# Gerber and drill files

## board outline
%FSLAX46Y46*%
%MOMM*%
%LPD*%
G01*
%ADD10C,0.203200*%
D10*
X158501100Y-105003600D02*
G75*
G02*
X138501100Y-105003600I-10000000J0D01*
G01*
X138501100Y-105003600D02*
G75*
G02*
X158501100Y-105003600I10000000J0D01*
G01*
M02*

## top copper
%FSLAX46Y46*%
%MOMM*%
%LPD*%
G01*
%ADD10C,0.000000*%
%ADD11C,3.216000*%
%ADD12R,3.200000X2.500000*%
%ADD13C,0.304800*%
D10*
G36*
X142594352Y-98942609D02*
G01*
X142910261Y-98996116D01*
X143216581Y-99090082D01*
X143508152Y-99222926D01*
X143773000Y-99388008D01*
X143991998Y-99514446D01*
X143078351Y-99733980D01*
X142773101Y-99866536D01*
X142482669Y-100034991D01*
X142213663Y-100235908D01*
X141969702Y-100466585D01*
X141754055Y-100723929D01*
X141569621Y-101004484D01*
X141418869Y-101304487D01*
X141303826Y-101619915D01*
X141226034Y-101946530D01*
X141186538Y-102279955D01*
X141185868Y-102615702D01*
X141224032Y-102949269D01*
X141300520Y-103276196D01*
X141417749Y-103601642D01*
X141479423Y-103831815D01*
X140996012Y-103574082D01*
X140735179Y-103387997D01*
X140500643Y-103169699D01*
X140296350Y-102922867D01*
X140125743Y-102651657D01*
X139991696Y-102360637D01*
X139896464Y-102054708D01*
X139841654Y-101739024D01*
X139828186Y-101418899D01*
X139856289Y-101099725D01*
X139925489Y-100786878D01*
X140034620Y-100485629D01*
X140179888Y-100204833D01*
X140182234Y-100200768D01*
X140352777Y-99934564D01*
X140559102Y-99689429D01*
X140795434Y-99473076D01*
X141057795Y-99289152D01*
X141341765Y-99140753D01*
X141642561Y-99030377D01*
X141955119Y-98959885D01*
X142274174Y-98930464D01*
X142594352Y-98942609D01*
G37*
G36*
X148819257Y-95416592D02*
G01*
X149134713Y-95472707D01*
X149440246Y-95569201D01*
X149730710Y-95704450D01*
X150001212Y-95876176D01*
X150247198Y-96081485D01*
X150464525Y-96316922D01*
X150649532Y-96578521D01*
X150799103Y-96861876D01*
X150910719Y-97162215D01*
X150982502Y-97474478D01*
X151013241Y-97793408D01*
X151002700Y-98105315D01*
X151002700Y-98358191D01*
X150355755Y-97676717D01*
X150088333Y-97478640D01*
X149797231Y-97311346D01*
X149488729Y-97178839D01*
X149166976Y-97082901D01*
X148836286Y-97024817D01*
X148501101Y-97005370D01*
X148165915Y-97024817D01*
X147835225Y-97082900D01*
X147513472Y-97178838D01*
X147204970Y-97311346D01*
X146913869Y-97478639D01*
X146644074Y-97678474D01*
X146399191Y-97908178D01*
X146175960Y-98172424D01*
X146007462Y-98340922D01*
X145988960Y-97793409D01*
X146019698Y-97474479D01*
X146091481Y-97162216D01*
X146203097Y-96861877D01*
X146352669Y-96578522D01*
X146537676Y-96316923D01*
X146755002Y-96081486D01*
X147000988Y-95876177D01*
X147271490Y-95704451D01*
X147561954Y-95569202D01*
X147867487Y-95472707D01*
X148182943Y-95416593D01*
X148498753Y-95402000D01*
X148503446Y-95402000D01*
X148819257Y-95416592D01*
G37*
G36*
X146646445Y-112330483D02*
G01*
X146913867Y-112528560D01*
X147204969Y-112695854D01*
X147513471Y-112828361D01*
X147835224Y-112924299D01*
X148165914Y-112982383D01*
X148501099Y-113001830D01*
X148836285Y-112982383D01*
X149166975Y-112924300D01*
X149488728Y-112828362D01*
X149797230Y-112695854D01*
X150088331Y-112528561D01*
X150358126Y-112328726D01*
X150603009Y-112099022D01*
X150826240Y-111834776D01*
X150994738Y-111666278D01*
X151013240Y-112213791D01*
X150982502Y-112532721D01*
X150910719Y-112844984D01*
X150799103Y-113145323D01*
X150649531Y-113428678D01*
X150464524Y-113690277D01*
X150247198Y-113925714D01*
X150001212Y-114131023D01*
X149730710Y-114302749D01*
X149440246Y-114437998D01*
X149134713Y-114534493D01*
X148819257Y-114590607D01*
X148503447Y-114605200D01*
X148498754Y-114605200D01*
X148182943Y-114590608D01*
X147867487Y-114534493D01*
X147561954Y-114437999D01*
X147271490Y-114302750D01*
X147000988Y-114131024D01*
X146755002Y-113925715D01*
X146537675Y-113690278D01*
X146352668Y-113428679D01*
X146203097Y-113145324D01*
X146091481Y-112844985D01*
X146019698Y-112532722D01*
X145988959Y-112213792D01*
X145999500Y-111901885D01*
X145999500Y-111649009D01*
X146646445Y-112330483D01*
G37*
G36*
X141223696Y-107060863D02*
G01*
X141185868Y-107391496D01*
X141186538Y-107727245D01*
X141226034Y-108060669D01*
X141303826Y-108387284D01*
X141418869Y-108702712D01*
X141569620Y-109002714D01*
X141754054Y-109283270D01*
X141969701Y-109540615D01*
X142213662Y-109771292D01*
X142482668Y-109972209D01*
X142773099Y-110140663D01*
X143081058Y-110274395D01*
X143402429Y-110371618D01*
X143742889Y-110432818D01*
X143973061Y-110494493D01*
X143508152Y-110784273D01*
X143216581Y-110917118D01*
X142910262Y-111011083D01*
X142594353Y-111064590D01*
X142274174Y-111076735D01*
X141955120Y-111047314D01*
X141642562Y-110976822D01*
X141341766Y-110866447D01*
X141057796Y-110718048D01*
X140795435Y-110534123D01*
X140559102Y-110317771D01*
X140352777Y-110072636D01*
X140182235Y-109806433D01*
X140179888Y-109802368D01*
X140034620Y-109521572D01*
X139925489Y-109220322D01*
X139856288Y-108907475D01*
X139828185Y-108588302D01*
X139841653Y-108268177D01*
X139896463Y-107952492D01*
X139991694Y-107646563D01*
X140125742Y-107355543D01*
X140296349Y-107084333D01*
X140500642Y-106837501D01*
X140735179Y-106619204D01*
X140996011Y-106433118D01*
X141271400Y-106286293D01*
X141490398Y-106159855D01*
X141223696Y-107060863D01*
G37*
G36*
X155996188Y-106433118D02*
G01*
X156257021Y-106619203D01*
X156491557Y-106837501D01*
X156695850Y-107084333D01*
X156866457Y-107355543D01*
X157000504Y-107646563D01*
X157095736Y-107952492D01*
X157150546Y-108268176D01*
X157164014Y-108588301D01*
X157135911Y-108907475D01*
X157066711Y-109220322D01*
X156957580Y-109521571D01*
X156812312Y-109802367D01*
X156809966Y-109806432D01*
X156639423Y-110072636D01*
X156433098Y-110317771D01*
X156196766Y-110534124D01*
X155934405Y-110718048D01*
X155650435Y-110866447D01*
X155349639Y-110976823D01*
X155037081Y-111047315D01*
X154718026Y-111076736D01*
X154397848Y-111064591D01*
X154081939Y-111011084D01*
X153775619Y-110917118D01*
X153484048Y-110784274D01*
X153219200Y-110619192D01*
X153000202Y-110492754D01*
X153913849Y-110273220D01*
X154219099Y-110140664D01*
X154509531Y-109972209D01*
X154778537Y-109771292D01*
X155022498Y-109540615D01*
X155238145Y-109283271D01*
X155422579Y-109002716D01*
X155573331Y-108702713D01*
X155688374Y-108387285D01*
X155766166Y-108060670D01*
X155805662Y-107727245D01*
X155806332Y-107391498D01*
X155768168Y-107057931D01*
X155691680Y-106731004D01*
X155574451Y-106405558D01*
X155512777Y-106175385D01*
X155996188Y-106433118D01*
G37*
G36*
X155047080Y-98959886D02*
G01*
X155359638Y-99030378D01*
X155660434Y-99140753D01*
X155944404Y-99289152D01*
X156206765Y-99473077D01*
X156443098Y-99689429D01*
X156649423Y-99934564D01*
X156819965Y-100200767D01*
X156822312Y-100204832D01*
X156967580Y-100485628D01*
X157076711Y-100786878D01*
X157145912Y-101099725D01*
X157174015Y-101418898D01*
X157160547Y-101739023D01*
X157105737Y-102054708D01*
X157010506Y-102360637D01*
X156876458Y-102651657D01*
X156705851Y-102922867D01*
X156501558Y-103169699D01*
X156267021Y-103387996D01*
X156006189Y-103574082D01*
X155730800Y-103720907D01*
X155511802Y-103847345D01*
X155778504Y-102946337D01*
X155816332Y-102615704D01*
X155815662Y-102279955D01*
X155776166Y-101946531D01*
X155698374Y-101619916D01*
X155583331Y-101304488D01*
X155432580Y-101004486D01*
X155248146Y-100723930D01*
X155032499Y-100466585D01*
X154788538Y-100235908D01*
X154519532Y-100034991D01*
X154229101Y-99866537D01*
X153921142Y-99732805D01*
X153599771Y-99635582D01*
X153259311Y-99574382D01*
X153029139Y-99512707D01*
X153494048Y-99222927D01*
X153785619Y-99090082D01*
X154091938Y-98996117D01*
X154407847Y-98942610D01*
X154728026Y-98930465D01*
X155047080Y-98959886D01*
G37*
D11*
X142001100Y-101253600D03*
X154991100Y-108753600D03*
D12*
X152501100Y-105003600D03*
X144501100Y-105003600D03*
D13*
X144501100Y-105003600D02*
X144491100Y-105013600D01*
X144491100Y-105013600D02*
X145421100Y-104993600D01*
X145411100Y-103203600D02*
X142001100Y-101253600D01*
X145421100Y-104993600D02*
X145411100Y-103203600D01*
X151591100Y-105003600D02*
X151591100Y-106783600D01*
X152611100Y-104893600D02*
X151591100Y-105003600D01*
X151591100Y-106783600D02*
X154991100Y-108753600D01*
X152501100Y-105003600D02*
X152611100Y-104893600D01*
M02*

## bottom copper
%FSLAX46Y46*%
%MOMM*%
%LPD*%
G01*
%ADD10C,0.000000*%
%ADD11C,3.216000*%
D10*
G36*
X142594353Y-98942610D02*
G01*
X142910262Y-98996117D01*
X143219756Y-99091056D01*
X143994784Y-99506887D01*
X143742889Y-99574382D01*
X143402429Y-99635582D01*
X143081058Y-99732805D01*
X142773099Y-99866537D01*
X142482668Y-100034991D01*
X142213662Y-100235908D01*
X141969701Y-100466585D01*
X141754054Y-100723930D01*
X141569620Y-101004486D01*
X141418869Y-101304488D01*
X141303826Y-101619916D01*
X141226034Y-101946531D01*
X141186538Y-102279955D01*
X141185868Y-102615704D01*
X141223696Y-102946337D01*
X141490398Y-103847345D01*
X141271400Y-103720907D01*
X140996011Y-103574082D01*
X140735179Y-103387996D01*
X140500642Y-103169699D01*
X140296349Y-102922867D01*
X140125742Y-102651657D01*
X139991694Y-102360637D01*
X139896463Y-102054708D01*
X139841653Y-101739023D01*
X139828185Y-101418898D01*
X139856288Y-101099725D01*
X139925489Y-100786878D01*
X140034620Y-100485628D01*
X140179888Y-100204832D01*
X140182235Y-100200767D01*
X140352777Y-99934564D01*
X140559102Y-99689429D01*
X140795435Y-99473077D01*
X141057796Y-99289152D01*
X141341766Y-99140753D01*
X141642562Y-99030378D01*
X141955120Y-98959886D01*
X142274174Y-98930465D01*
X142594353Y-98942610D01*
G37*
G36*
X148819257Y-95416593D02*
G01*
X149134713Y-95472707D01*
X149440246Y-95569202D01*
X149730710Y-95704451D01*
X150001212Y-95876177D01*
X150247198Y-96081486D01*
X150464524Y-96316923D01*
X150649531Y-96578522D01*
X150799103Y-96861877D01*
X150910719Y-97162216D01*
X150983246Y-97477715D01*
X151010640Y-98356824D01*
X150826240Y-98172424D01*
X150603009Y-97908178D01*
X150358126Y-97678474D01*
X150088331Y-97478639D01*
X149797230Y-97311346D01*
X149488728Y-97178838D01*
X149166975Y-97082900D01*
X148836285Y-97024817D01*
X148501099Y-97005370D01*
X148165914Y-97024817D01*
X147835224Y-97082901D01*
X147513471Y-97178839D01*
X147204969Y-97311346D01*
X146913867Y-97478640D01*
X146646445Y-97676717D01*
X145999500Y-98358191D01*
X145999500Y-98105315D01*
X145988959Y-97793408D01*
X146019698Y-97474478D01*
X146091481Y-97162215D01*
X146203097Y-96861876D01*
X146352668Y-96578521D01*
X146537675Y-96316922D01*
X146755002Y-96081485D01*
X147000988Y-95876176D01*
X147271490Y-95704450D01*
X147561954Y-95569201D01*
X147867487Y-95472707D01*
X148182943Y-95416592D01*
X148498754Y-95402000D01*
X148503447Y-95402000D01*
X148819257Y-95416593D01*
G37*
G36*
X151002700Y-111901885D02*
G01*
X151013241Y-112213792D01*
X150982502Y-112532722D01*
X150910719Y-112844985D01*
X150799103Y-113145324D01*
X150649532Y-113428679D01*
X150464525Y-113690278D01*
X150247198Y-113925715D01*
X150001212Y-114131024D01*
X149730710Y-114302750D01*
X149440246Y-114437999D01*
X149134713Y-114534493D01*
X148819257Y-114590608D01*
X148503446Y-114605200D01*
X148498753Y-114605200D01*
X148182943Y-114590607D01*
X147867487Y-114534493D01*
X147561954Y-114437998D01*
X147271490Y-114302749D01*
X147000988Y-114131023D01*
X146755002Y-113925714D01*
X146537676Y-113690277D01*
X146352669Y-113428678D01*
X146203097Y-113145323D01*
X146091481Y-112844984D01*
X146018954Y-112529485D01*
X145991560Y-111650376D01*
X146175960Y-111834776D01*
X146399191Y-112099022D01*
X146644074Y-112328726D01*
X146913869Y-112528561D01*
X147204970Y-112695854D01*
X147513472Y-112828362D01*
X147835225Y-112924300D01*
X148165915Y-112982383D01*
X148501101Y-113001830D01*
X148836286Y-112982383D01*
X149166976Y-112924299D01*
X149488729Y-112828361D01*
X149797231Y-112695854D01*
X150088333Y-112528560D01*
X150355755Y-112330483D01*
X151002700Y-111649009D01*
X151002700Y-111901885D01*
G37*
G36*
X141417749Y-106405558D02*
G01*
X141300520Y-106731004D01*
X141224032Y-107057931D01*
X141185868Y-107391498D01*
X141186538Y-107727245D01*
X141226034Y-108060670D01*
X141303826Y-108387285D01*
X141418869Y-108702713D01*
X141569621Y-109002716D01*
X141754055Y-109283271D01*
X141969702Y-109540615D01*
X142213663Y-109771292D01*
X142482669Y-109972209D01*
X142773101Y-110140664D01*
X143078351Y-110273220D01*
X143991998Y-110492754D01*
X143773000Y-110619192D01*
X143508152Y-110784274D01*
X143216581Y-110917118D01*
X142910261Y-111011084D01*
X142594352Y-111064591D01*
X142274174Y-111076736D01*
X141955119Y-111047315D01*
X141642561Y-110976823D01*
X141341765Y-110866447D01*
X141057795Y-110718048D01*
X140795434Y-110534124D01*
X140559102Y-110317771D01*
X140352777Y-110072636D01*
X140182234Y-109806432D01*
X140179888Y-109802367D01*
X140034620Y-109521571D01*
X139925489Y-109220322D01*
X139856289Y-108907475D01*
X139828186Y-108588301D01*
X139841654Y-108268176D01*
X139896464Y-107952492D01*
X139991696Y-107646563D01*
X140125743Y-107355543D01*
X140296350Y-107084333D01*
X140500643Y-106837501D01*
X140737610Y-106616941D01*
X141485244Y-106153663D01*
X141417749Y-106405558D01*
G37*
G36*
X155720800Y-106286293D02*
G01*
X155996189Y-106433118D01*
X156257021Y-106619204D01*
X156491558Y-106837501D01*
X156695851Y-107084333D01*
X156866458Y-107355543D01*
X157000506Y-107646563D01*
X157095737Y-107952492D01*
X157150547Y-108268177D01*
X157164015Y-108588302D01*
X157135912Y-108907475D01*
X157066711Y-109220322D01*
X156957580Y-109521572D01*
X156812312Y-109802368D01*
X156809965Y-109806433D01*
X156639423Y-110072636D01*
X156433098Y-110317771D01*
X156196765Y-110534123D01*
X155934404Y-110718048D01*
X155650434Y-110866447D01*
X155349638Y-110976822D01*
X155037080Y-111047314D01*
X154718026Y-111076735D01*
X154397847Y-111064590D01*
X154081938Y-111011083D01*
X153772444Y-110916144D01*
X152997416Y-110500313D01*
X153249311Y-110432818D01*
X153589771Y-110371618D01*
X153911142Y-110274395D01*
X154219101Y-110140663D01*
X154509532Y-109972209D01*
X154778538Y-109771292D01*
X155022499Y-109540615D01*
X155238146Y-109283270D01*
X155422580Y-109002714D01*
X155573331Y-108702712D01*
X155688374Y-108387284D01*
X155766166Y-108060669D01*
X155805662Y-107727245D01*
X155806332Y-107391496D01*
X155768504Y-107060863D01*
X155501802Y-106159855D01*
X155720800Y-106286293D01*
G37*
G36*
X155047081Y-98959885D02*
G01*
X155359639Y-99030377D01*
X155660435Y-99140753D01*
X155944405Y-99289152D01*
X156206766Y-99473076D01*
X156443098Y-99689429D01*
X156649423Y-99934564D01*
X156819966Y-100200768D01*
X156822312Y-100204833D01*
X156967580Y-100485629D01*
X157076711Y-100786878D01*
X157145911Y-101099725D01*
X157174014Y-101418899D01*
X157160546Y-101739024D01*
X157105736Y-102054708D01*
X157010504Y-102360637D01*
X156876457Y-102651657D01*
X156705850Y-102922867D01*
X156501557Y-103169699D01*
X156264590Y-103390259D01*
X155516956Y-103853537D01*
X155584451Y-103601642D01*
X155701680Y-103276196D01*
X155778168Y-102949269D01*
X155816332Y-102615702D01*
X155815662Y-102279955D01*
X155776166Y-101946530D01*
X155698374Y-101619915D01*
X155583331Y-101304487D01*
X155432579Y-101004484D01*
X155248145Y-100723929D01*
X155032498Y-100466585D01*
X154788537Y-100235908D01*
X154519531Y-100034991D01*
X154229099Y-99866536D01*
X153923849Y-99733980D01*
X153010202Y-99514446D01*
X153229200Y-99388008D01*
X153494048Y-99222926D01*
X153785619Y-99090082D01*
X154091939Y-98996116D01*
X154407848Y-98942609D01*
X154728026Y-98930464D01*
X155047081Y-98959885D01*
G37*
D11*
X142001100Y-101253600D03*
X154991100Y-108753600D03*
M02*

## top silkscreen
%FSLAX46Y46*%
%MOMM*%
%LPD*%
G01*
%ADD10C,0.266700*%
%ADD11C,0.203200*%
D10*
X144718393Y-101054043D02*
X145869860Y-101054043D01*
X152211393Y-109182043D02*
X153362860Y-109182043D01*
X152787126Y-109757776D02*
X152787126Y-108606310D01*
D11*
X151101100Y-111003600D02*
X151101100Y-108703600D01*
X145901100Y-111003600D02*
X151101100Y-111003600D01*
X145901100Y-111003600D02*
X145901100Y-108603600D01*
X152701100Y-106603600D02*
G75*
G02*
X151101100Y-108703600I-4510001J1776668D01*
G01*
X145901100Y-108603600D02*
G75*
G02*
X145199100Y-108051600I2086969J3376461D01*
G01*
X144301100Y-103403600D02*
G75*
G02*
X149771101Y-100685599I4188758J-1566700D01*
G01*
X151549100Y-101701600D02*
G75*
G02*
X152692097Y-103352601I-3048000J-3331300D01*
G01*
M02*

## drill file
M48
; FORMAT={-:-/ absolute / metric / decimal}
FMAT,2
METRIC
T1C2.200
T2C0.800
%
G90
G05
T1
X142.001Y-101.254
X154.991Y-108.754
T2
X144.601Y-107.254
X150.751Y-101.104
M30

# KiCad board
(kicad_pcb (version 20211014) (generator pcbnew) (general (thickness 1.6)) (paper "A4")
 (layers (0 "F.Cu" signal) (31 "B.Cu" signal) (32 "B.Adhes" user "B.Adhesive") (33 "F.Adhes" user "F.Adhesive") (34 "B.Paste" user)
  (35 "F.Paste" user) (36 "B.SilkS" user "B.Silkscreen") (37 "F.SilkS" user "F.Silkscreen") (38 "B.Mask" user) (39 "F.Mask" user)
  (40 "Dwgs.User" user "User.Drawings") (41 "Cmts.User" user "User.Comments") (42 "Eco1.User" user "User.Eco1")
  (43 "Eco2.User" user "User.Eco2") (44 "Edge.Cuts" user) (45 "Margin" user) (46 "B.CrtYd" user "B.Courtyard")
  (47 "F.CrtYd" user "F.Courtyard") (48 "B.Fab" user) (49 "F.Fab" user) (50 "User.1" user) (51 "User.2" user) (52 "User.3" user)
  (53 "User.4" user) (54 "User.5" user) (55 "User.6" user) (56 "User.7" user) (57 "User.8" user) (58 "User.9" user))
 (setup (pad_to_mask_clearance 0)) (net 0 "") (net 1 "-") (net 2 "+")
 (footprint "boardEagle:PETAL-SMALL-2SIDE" (layer "F.Cu") (at 142.0011 101.2536 -120)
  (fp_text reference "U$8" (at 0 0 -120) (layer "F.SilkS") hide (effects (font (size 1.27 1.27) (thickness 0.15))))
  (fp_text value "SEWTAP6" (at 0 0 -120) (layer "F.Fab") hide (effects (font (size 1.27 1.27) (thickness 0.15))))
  (fp_poly
   (pts (xy -1.854655 -0.173117) (xy -1.587233 0.02496) (xy -1.296131 0.192254) (xy -0.987629 0.324761) (xy -0.665876 0.420699)
    (xy -0.335186 0.478783) (xy -0.000001 0.49823) (xy 0.335185 0.478783) (xy 0.665875 0.4207) (xy 0.987628 0.324762) (xy 1.29613 0.192254)
    (xy 1.587231 0.024961) (xy 1.857026 -0.174874) (xy 2.101909 -0.404578) (xy 2.32514 -0.668824) (xy 2.493638 -0.837322)
    (xy 2.51214 -0.289809) (xy 2.481402 0.029121) (xy 2.409619 0.341384) (xy 2.298003 0.641723) (xy 2.148431 0.925078)
    (xy 1.963424 1.186677) (xy 1.746098 1.422114) (xy 1.500112 1.627423) (xy 1.22961 1.799149) (xy 0.939146 1.934398) (xy 0.633613 2.030893)
    (xy 0.318157 2.087007) (xy 0.002347 2.1016) (xy -0.002346 2.1016) (xy -0.318157 2.087008) (xy -0.633613 2.030893)
    (xy -0.939146 1.934399) (xy -1.22961 1.79915) (xy -1.500112 1.627424) (xy -1.746098 1.422115) (xy -1.963425 1.186678)
    (xy -2.148432 0.925079) (xy -2.298003 0.641724) (xy -2.409619 0.341385) (xy -2.481402 0.029122) (xy -2.512141 -0.289808)
    (xy -2.5016 -0.601715) (xy -2.5016 -0.854591))
   (layer "F.Cu") (width 0) (fill solid))
  (fp_poly
   (pts (xy 2.5016 -0.601715) (xy 2.512141 -0.289808) (xy 2.481402 0.029122) (xy 2.409619 0.341385) (xy 2.298003 0.641724)
    (xy 2.148432 0.925079) (xy 1.963425 1.186678) (xy 1.746098 1.422115) (xy 1.500112 1.627424) (xy 1.22961 1.79915) (xy 0.939146 1.934399)
    (xy 0.633613 2.030893) (xy 0.318157 2.087008) (xy 0.002346 2.1016) (xy -0.002347 2.1016) (xy -0.318157 2.087007) (xy -0.633613 2.030893)
    (xy -0.939146 1.934398) (xy -1.22961 1.799149) (xy -1.500112 1.627423) (xy -1.746098 1.422114) (xy -1.963424 1.186677)
    (xy -2.148431 0.925078) (xy -2.298003 0.641723) (xy -2.409619 0.341384) (xy -2.482146 0.025885) (xy -2.50954 -0.853224)
    (xy -2.32514 -0.668824) (xy -2.101909 -0.404578) (xy -1.857026 -0.174874) (xy -1.587231 0.024961) (xy -1.29613 0.192254)
    (xy -0.987628 0.324762) (xy -0.665875 0.4207) (xy -0.335185 0.478783) (xy 0.000001 0.49823) (xy 0.335186 0.478783)
    (xy 0.665876 0.420699) (xy 0.987629 0.324761) (xy 1.296131 0.192254) (xy 1.587233 0.02496) (xy 1.854655 -0.173117) (xy 2.5016 -0.854591))
   (layer "B.Cu") (width 0) (fill solid))
  (pad "1" thru_hole circle (at 0 0 330) (size 3.216 3.216) (drill 2.2) (layers *.Cu *.Mask) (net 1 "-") (solder_mask_margin 0.1016)))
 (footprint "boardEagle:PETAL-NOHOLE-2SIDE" (layer "F.Cu") (at 148.5011 97.5036 180)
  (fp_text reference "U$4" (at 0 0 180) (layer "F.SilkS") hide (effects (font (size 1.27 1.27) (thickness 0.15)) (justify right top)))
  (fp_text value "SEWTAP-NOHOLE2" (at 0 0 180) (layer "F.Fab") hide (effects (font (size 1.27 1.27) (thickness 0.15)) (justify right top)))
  (fp_poly
   (pts (xy -1.854655 -0.173117) (xy -1.587233 0.02496) (xy -1.296131 0.192254) (xy -0.987629 0.324761) (xy -0.665876 0.420699)
    (xy -0.335186 0.478783) (xy -0.000001 0.49823) (xy 0.335185 0.478783) (xy 0.665875 0.4207) (xy 0.987628 0.324762) (xy 1.29613 0.192254)
    (xy 1.587231 0.024961) (xy 1.857026 -0.174874) (xy 2.101909 -0.404578) (xy 2.32514 -0.668824) (xy 2.493638 -0.837322)
    (xy 2.51214 -0.289809) (xy 2.481402 0.029121) (xy 2.409619 0.341384) (xy 2.298003 0.641723) (xy 2.148431 0.925078)
    (xy 1.963424 1.186677) (xy 1.746098 1.422114) (xy 1.500112 1.627423) (xy 1.22961 1.799149) (xy 0.939146 1.934398) (xy 0.633613 2.030893)
    (xy 0.318157 2.087007) (xy 0.002347 2.1016) (xy -0.002346 2.1016) (xy -0.318157 2.087008) (xy -0.633613 2.030893)
    (xy -0.939146 1.934399) (xy -1.22961 1.79915) (xy -1.500112 1.627424) (xy -1.746098 1.422115) (xy -1.963425 1.186678)
    (xy -2.148432 0.925079) (xy -2.298003 0.641724) (xy -2.409619 0.341385) (xy -2.481402 0.029122) (xy -2.512141 -0.289808)
    (xy -2.5016 -0.601715) (xy -2.5016 -0.854591))
   (layer "F.Cu") (width 0) (fill solid))
  (fp_poly
   (pts (xy 2.5016 -0.601715) (xy 2.512141 -0.289808) (xy 2.481402 0.029122) (xy 2.409619 0.341385) (xy 2.298003 0.641724)
    (xy 2.148432 0.925079) (xy 1.963425 1.186678) (xy 1.746098 1.422115) (xy 1.500112 1.627424) (xy 1.22961 1.79915) (xy 0.939146 1.934399)
    (xy 0.633613 2.030893) (xy 0.318157 2.087008) (xy 0.002346 2.1016) (xy -0.002347 2.1016) (xy -0.318157 2.087007) (xy -0.633613 2.030893)
    (xy -0.939146 1.934398) (xy -1.22961 1.799149) (xy -1.500112 1.627423) (xy -1.746098 1.422114) (xy -1.963424 1.186677)
    (xy -2.148431 0.925078) (xy -2.298003 0.641723) (xy -2.409619 0.341384) (xy -2.482146 0.025885) (xy -2.50954 -0.853224)
    (xy -2.32514 -0.668824) (xy -2.101909 -0.404578) (xy -1.857026 -0.174874) (xy -1.587231 0.024961) (xy -1.29613 0.192254)
    (xy -0.987628 0.324762) (xy -0.665875 0.4207) (xy -0.335185 0.478783) (xy 0.000001 0.49823) (xy 0.335186 0.478783)
    (xy 0.665876 0.420699) (xy 0.987629 0.324761) (xy 1.296131 0.192254) (xy 1.587233 0.02496) (xy 1.854655 -0.173117) (xy 2.5016 -0.854591))
   (layer "B.Cu") (width 0) (fill solid)))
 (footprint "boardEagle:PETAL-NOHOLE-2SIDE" (layer "F.Cu") (at 148.5011 112.5036)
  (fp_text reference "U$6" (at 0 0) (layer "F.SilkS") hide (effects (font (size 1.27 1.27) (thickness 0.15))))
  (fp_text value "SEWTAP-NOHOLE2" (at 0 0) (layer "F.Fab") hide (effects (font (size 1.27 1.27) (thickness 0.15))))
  (fp_poly
   (pts (xy -1.854655 -0.173117) (xy -1.587233 0.02496) (xy -1.296131 0.192254) (xy -0.987629 0.324761) (xy -0.665876 0.420699)
    (xy -0.335186 0.478783) (xy -0.000001 0.49823) (xy 0.335185 0.478783) (xy 0.665875 0.4207) (xy 0.987628 0.324762) (xy 1.29613 0.192254)
    (xy 1.587231 0.024961) (xy 1.857026 -0.174874) (xy 2.101909 -0.404578) (xy 2.32514 -0.668824) (xy 2.493638 -0.837322)
    (xy 2.51214 -0.289809) (xy 2.481402 0.029121) (xy 2.409619 0.341384) (xy 2.298003 0.641723) (xy 2.148431 0.925078)
    (xy 1.963424 1.186677) (xy 1.746098 1.422114) (xy 1.500112 1.627423) (xy 1.22961 1.799149) (xy 0.939146 1.934398) (xy 0.633613 2.030893)
    (xy 0.318157 2.087007) (xy 0.002347 2.1016) (xy -0.002346 2.1016) (xy -0.318157 2.087008) (xy -0.633613 2.030893)
    (xy -0.939146 1.934399) (xy -1.22961 1.79915) (xy -1.500112 1.627424) (xy -1.746098 1.422115) (xy -1.963425 1.186678)
    (xy -2.148432 0.925079) (xy -2.298003 0.641724) (xy -2.409619 0.341385) (xy -2.481402 0.029122) (xy -2.512141 -0.289808)
    (xy -2.5016 -0.601715) (xy -2.5016 -0.854591))
   (layer "F.Cu") (width 0) (fill solid))
  (fp_poly
   (pts (xy 2.5016 -0.601715) (xy 2.512141 -0.289808) (xy 2.481402 0.029122) (xy 2.409619 0.341385) (xy 2.298003 0.641724)
    (xy 2.148432 0.925079) (xy 1.963425 1.186678) (xy 1.746098 1.422115) (xy 1.500112 1.627424) (xy 1.22961 1.79915) (xy 0.939146 1.934399)
    (xy 0.633613 2.030893) (xy 0.318157 2.087008) (xy 0.002346 2.1016) (xy -0.002347 2.1016) (xy -0.318157 2.087007) (xy -0.633613 2.030893)
    (xy -0.939146 1.934398) (xy -1.22961 1.799149) (xy -1.500112 1.627423) (xy -1.746098 1.422114) (xy -1.963424 1.186677)
    (xy -2.148431 0.925078) (xy -2.298003 0.641723) (xy -2.409619 0.341384) (xy -2.482146 0.025885) (xy -2.50954 -0.853224)
    (xy -2.32514 -0.668824) (xy -2.101909 -0.404578) (xy -1.857026 -0.174874) (xy -1.587231 0.024961) (xy -1.29613 0.192254)
    (xy -0.987628 0.324762) (xy -0.665875 0.4207) (xy -0.335185 0.478783) (xy 0.000001 0.49823) (xy 0.335186 0.478783)
    (xy 0.665876 0.420699) (xy 0.987629 0.324761) (xy 1.296131 0.192254) (xy 1.587233 0.02496) (xy 1.854655 -0.173117) (xy 2.5016 -0.854591))
   (layer "B.Cu") (width 0) (fill solid)))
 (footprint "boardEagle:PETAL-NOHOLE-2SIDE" (layer "F.Cu") (at 142.0011 108.7536 -60)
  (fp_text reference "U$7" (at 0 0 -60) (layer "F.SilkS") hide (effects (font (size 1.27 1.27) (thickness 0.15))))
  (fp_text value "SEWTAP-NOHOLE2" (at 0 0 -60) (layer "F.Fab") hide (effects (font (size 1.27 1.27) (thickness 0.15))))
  (fp_poly
   (pts (xy -1.854655 -0.173117) (xy -1.587233 0.02496) (xy -1.296131 0.192254) (xy -0.987629 0.324761) (xy -0.665876 0.420699)
    (xy -0.335186 0.478783) (xy -0.000001 0.49823) (xy 0.335185 0.478783) (xy 0.665875 0.4207) (xy 0.987628 0.324762) (xy 1.29613 0.192254)
    (xy 1.587231 0.024961) (xy 1.857026 -0.174874) (xy 2.101909 -0.404578) (xy 2.32514 -0.668824) (xy 2.493638 -0.837322)
    (xy 2.51214 -0.289809) (xy 2.481402 0.029121) (xy 2.409619 0.341384) (xy 2.298003 0.641723) (xy 2.148431 0.925078)
    (xy 1.963424 1.186677) (xy 1.746098 1.422114) (xy 1.500112 1.627423) (xy 1.22961 1.799149) (xy 0.939146 1.934398) (xy 0.633613 2.030893)
    (xy 0.318157 2.087007) (xy 0.002347 2.1016) (xy -0.002346 2.1016) (xy -0.318157 2.087008) (xy -0.633613 2.030893)
    (xy -0.939146 1.934399) (xy -1.22961 1.79915) (xy -1.500112 1.627424) (xy -1.746098 1.422115) (xy -1.963425 1.186678)
    (xy -2.148432 0.925079) (xy -2.298003 0.641724) (xy -2.409619 0.341385) (xy -2.481402 0.029122) (xy -2.512141 -0.289808)
    (xy -2.5016 -0.601715) (xy -2.5016 -0.854591))
   (layer "F.Cu") (width 0) (fill solid))
  (fp_poly
   (pts (xy 2.5016 -0.601715) (xy 2.512141 -0.289808) (xy 2.481402 0.029122) (xy 2.409619 0.341385) (xy 2.298003 0.641724)
    (xy 2.148432 0.925079) (xy 1.963425 1.186678) (xy 1.746098 1.422115) (xy 1.500112 1.627424) (xy 1.22961 1.79915) (xy 0.939146 1.934399)
    (xy 0.633613 2.030893) (xy 0.318157 2.087008) (xy 0.002346 2.1016) (xy -0.002347 2.1016) (xy -0.318157 2.087007) (xy -0.633613 2.030893)
    (xy -0.939146 1.934398) (xy -1.22961 1.799149) (xy -1.500112 1.627423) (xy -1.746098 1.422114) (xy -1.963424 1.186677)
    (xy -2.148431 0.925078) (xy -2.298003 0.641723) (xy -2.409619 0.341384) (xy -2.482146 0.025885) (xy -2.50954 -0.853224)
    (xy -2.32514 -0.668824) (xy -2.101909 -0.404578) (xy -1.857026 -0.174874) (xy -1.587231 0.024961) (xy -1.29613 0.192254)
    (xy -0.987628 0.324762) (xy -0.665875 0.4207) (xy -0.335185 0.478783) (xy 0.000001 0.49823) (xy 0.335186 0.478783)
    (xy 0.665876 0.420699) (xy 0.987629 0.324761) (xy 1.296131 0.192254) (xy 1.587233 0.02496) (xy 1.854655 -0.173117) (xy 2.5016 -0.854591))
   (layer "B.Cu") (width 0) (fill solid)))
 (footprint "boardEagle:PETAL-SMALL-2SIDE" (layer "F.Cu") (at 154.9911 108.7536 60)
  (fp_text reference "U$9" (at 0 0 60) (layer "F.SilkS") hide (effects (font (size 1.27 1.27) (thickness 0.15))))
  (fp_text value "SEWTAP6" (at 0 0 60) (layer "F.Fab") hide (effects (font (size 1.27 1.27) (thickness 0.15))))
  (fp_poly
   (pts (xy -1.854655 -0.173117) (xy -1.587233 0.02496) (xy -1.296131 0.192254) (xy -0.987629 0.324761) (xy -0.665876 0.420699)
    (xy -0.335186 0.478783) (xy -0.000001 0.49823) (xy 0.335185 0.478783) (xy 0.665875 0.4207) (xy 0.987628 0.324762) (xy 1.29613 0.192254)
    (xy 1.587231 0.024961) (xy 1.857026 -0.174874) (xy 2.101909 -0.404578) (xy 2.32514 -0.668824) (xy 2.493638 -0.837322)
    (xy 2.51214 -0.289809) (xy 2.481402 0.029121) (xy 2.409619 0.341384) (xy 2.298003 0.641723) (xy 2.148431 0.925078)
    (xy 1.963424 1.186677) (xy 1.746098 1.422114) (xy 1.500112 1.627423) (xy 1.22961 1.799149) (xy 0.939146 1.934398) (xy 0.633613 2.030893)
    (xy 0.318157 2.087007) (xy 0.002347 2.1016) (xy -0.002346 2.1016) (xy -0.318157 2.087008) (xy -0.633613 2.030893)
    (xy -0.939146 1.934399) (xy -1.22961 1.79915) (xy -1.500112 1.627424) (xy -1.746098 1.422115) (xy -1.963425 1.186678)
    (xy -2.148432 0.925079) (xy -2.298003 0.641724) (xy -2.409619 0.341385) (xy -2.481402 0.029122) (xy -2.512141 -0.289808)
    (xy -2.5016 -0.601715) (xy -2.5016 -0.854591))
   (layer "F.Cu") (width 0) (fill solid))
  (fp_poly
   (pts (xy 2.5016 -0.601715) (xy 2.512141 -0.289808) (xy 2.481402 0.029122) (xy 2.409619 0.341385) (xy 2.298003 0.641724)
    (xy 2.148432 0.925079) (xy 1.963425 1.186678) (xy 1.746098 1.422115) (xy 1.500112 1.627424) (xy 1.22961 1.79915) (xy 0.939146 1.934399)
    (xy 0.633613 2.030893) (xy 0.318157 2.087008) (xy 0.002346 2.1016) (xy -0.002347 2.1016) (xy -0.318157 2.087007) (xy -0.633613 2.030893)
    (xy -0.939146 1.934398) (xy -1.22961 1.799149) (xy -1.500112 1.627423) (xy -1.746098 1.422114) (xy -1.963424 1.186677)
    (xy -2.148431 0.925078) (xy -2.298003 0.641723) (xy -2.409619 0.341384) (xy -2.482146 0.025885) (xy -2.50954 -0.853224)
    (xy -2.32514 -0.668824) (xy -2.101909 -0.404578) (xy -1.857026 -0.174874) (xy -1.587231 0.024961) (xy -1.29613 0.192254)
    (xy -0.987628 0.324762) (xy -0.665875 0.4207) (xy -0.335185 0.478783) (xy 0.000001 0.49823) (xy 0.335186 0.478783)
    (xy 0.665876 0.420699) (xy 0.987629 0.324761) (xy 1.296131 0.192254) (xy 1.587233 0.02496) (xy 1.854655 -0.173117) (xy 2.5016 -0.854591))
   (layer "B.Cu") (width 0) (fill solid))
  (pad "1" thru_hole circle (at 0 0 150) (size 3.216 3.216) (drill 2.2) (layers *.Cu *.Mask) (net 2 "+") (solder_mask_margin 0.1016)))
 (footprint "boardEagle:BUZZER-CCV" (layer "F.Cu") (at 148.5011 105.0036)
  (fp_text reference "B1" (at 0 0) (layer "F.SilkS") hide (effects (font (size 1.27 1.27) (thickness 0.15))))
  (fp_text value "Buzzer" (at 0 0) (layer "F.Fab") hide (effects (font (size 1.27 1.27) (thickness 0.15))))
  (fp_line (start 2.6 6) (end 2.6 3.7) (layer "F.SilkS") (width 0.2032))
  (fp_line (start -2.6 6) (end 2.6 6) (layer "F.SilkS") (width 0.2032))
  (fp_line (start -2.6 6) (end -2.6 3.6) (layer "F.SilkS") (width 0.2032))
  (fp_arc (start 4.2 1.6) (mid 3.545723 2.761027) (end 2.6 3.7) (layer "F.SilkS") (width 0.2032))
  (fp_arc (start -2.6 3.6) (mid -2.966573 3.343805) (end -3.302 3.048) (layer "F.SilkS") (width 0.2032))
  (fp_arc (start -4.2 -1.6) (mid -2.00129 -4.038291) (end 1.270001 -4.318001) (layer "F.SilkS") (width 0.2032))
  (fp_arc (start 3.048 -3.302) (mid 3.712443 -2.540845) (end 4.191 -1.651) (layer "F.SilkS") (width 0.2032))
  (pad "" np_thru_hole circle (at -3.9 2.25) (size 0.8 0.8) (drill 0.8) (layers *.Cu *.Mask))
  (pad "" np_thru_hole circle (at 2.25 -3.9) (size 0.8 0.8) (drill 0.8) (layers *.Cu *.Mask))
  (pad "+" smd rect (at 4 0) (size 3.2 2.5) (layers "F.Cu" "F.Paste" "F.Mask") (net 2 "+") (solder_mask_margin 0.1016))
  (pad "-" smd rect (at -4 0) (size 3.2 2.5) (layers "F.Cu" "F.Paste" "F.Mask") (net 1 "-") (solder_mask_margin 0.1016)))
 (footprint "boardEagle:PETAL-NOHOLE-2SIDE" (layer "F.Cu") (at 155.0011 101.2536 120)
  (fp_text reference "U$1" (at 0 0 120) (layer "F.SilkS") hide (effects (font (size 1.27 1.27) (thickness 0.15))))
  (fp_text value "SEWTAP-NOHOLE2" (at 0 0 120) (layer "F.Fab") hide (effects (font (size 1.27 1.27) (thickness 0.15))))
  (fp_poly
   (pts (xy -1.854655 -0.173117) (xy -1.587233 0.02496) (xy -1.296131 0.192254) (xy -0.987629 0.324761) (xy -0.665876 0.420699)
    (xy -0.335186 0.478783) (xy -0.000001 0.49823) (xy 0.335185 0.478783) (xy 0.665875 0.4207) (xy 0.987628 0.324762) (xy 1.29613 0.192254)
    (xy 1.587231 0.024961) (xy 1.857026 -0.174874) (xy 2.101909 -0.404578) (xy 2.32514 -0.668824) (xy 2.493638 -0.837322)
    (xy 2.51214 -0.289809) (xy 2.481402 0.029121) (xy 2.409619 0.341384) (xy 2.298003 0.641723) (xy 2.148431 0.925078)
    (xy 1.963424 1.186677) (xy 1.746098 1.422114) (xy 1.500112 1.627423) (xy 1.22961 1.799149) (xy 0.939146 1.934398) (xy 0.633613 2.030893)
    (xy 0.318157 2.087007) (xy 0.002347 2.1016) (xy -0.002346 2.1016) (xy -0.318157 2.087008) (xy -0.633613 2.030893)
    (xy -0.939146 1.934399) (xy -1.22961 1.79915) (xy -1.500112 1.627424) (xy -1.746098 1.422115) (xy -1.963425 1.186678)
    (xy -2.148432 0.925079) (xy -2.298003 0.641724) (xy -2.409619 0.341385) (xy -2.481402 0.029122) (xy -2.512141 -0.289808)
    (xy -2.5016 -0.601715) (xy -2.5016 -0.854591))
   (layer "F.Cu") (width 0) (fill solid))
  (fp_poly
   (pts (xy 2.5016 -0.601715) (xy 2.512141 -0.289808) (xy 2.481402 0.029122) (xy 2.409619 0.341385) (xy 2.298003 0.641724)
    (xy 2.148432 0.925079) (xy 1.963425 1.186678) (xy 1.746098 1.422115) (xy 1.500112 1.627424) (xy 1.22961 1.79915) (xy 0.939146 1.934399)
    (xy 0.633613 2.030893) (xy 0.318157 2.087008) (xy 0.002346 2.1016) (xy -0.002347 2.1016) (xy -0.318157 2.087007) (xy -0.633613 2.030893)
    (xy -0.939146 1.934398) (xy -1.22961 1.799149) (xy -1.500112 1.627423) (xy -1.746098 1.422114) (xy -1.963424 1.186677)
    (xy -2.148431 0.925078) (xy -2.298003 0.641723) (xy -2.409619 0.341384) (xy -2.482146 0.025885) (xy -2.50954 -0.853224)
    (xy -2.32514 -0.668824) (xy -2.101909 -0.404578) (xy -1.857026 -0.174874) (xy -1.587231 0.024961) (xy -1.29613 0.192254)
    (xy -0.987628 0.324762) (xy -0.665875 0.4207) (xy -0.335185 0.478783) (xy 0.000001 0.49823) (xy 0.335186 0.478783)
    (xy 0.665876 0.420699) (xy 0.987629 0.324761) (xy 1.296131 0.192254) (xy 1.587233 0.02496) (xy 1.854655 -0.173117) (xy 2.5016 -0.854591))
   (layer "B.Cu") (width 0) (fill solid)))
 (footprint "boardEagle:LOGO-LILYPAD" (layer "B.Cu") (at 148.5011 105.0036 180)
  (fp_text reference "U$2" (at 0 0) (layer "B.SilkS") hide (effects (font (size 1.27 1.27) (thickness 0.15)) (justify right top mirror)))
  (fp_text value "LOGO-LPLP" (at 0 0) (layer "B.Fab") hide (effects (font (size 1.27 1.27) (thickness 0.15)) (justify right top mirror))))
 (gr_circle (center 148.5011 105.0036) (end 158.5011 105.0036) (layer "Edge.Cuts") (width 0.2032) (fill none))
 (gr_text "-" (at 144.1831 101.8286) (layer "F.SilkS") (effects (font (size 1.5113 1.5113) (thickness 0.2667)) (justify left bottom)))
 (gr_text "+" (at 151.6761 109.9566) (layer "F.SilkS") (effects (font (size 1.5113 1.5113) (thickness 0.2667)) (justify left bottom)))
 (segment (start 144.5011 105.0036) (end 144.4911 105.0136) (width 0.3048) (layer "F.Cu") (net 1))
 (segment (start 144.4911 105.0136) (end 145.4211 104.9936) (width 0.3048) (layer "F.Cu") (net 1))
 (segment (start 145.4111 103.2036) (end 142.0011 101.2536) (width 0.3048) (layer "F.Cu") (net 1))
 (segment (start 145.4211 104.9936) (end 145.4111 103.2036) (width 0.3048) (layer "F.Cu") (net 1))
 (segment (start 151.5911 105.0036) (end 151.5911 106.7836) (width 0.3048) (layer "F.Cu") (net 2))
 (segment (start 152.6111 104.8936) (end 151.5911 105.0036) (width 0.3048) (layer "F.Cu") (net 2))
 (segment (start 151.5911 106.7836) (end 154.9911 108.7536) (width 0.3048) (layer "F.Cu") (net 2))
 (segment (start 152.5011 105.0036) (end 152.6111 104.8936) (width 0.3048) (layer "F.Cu") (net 2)))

